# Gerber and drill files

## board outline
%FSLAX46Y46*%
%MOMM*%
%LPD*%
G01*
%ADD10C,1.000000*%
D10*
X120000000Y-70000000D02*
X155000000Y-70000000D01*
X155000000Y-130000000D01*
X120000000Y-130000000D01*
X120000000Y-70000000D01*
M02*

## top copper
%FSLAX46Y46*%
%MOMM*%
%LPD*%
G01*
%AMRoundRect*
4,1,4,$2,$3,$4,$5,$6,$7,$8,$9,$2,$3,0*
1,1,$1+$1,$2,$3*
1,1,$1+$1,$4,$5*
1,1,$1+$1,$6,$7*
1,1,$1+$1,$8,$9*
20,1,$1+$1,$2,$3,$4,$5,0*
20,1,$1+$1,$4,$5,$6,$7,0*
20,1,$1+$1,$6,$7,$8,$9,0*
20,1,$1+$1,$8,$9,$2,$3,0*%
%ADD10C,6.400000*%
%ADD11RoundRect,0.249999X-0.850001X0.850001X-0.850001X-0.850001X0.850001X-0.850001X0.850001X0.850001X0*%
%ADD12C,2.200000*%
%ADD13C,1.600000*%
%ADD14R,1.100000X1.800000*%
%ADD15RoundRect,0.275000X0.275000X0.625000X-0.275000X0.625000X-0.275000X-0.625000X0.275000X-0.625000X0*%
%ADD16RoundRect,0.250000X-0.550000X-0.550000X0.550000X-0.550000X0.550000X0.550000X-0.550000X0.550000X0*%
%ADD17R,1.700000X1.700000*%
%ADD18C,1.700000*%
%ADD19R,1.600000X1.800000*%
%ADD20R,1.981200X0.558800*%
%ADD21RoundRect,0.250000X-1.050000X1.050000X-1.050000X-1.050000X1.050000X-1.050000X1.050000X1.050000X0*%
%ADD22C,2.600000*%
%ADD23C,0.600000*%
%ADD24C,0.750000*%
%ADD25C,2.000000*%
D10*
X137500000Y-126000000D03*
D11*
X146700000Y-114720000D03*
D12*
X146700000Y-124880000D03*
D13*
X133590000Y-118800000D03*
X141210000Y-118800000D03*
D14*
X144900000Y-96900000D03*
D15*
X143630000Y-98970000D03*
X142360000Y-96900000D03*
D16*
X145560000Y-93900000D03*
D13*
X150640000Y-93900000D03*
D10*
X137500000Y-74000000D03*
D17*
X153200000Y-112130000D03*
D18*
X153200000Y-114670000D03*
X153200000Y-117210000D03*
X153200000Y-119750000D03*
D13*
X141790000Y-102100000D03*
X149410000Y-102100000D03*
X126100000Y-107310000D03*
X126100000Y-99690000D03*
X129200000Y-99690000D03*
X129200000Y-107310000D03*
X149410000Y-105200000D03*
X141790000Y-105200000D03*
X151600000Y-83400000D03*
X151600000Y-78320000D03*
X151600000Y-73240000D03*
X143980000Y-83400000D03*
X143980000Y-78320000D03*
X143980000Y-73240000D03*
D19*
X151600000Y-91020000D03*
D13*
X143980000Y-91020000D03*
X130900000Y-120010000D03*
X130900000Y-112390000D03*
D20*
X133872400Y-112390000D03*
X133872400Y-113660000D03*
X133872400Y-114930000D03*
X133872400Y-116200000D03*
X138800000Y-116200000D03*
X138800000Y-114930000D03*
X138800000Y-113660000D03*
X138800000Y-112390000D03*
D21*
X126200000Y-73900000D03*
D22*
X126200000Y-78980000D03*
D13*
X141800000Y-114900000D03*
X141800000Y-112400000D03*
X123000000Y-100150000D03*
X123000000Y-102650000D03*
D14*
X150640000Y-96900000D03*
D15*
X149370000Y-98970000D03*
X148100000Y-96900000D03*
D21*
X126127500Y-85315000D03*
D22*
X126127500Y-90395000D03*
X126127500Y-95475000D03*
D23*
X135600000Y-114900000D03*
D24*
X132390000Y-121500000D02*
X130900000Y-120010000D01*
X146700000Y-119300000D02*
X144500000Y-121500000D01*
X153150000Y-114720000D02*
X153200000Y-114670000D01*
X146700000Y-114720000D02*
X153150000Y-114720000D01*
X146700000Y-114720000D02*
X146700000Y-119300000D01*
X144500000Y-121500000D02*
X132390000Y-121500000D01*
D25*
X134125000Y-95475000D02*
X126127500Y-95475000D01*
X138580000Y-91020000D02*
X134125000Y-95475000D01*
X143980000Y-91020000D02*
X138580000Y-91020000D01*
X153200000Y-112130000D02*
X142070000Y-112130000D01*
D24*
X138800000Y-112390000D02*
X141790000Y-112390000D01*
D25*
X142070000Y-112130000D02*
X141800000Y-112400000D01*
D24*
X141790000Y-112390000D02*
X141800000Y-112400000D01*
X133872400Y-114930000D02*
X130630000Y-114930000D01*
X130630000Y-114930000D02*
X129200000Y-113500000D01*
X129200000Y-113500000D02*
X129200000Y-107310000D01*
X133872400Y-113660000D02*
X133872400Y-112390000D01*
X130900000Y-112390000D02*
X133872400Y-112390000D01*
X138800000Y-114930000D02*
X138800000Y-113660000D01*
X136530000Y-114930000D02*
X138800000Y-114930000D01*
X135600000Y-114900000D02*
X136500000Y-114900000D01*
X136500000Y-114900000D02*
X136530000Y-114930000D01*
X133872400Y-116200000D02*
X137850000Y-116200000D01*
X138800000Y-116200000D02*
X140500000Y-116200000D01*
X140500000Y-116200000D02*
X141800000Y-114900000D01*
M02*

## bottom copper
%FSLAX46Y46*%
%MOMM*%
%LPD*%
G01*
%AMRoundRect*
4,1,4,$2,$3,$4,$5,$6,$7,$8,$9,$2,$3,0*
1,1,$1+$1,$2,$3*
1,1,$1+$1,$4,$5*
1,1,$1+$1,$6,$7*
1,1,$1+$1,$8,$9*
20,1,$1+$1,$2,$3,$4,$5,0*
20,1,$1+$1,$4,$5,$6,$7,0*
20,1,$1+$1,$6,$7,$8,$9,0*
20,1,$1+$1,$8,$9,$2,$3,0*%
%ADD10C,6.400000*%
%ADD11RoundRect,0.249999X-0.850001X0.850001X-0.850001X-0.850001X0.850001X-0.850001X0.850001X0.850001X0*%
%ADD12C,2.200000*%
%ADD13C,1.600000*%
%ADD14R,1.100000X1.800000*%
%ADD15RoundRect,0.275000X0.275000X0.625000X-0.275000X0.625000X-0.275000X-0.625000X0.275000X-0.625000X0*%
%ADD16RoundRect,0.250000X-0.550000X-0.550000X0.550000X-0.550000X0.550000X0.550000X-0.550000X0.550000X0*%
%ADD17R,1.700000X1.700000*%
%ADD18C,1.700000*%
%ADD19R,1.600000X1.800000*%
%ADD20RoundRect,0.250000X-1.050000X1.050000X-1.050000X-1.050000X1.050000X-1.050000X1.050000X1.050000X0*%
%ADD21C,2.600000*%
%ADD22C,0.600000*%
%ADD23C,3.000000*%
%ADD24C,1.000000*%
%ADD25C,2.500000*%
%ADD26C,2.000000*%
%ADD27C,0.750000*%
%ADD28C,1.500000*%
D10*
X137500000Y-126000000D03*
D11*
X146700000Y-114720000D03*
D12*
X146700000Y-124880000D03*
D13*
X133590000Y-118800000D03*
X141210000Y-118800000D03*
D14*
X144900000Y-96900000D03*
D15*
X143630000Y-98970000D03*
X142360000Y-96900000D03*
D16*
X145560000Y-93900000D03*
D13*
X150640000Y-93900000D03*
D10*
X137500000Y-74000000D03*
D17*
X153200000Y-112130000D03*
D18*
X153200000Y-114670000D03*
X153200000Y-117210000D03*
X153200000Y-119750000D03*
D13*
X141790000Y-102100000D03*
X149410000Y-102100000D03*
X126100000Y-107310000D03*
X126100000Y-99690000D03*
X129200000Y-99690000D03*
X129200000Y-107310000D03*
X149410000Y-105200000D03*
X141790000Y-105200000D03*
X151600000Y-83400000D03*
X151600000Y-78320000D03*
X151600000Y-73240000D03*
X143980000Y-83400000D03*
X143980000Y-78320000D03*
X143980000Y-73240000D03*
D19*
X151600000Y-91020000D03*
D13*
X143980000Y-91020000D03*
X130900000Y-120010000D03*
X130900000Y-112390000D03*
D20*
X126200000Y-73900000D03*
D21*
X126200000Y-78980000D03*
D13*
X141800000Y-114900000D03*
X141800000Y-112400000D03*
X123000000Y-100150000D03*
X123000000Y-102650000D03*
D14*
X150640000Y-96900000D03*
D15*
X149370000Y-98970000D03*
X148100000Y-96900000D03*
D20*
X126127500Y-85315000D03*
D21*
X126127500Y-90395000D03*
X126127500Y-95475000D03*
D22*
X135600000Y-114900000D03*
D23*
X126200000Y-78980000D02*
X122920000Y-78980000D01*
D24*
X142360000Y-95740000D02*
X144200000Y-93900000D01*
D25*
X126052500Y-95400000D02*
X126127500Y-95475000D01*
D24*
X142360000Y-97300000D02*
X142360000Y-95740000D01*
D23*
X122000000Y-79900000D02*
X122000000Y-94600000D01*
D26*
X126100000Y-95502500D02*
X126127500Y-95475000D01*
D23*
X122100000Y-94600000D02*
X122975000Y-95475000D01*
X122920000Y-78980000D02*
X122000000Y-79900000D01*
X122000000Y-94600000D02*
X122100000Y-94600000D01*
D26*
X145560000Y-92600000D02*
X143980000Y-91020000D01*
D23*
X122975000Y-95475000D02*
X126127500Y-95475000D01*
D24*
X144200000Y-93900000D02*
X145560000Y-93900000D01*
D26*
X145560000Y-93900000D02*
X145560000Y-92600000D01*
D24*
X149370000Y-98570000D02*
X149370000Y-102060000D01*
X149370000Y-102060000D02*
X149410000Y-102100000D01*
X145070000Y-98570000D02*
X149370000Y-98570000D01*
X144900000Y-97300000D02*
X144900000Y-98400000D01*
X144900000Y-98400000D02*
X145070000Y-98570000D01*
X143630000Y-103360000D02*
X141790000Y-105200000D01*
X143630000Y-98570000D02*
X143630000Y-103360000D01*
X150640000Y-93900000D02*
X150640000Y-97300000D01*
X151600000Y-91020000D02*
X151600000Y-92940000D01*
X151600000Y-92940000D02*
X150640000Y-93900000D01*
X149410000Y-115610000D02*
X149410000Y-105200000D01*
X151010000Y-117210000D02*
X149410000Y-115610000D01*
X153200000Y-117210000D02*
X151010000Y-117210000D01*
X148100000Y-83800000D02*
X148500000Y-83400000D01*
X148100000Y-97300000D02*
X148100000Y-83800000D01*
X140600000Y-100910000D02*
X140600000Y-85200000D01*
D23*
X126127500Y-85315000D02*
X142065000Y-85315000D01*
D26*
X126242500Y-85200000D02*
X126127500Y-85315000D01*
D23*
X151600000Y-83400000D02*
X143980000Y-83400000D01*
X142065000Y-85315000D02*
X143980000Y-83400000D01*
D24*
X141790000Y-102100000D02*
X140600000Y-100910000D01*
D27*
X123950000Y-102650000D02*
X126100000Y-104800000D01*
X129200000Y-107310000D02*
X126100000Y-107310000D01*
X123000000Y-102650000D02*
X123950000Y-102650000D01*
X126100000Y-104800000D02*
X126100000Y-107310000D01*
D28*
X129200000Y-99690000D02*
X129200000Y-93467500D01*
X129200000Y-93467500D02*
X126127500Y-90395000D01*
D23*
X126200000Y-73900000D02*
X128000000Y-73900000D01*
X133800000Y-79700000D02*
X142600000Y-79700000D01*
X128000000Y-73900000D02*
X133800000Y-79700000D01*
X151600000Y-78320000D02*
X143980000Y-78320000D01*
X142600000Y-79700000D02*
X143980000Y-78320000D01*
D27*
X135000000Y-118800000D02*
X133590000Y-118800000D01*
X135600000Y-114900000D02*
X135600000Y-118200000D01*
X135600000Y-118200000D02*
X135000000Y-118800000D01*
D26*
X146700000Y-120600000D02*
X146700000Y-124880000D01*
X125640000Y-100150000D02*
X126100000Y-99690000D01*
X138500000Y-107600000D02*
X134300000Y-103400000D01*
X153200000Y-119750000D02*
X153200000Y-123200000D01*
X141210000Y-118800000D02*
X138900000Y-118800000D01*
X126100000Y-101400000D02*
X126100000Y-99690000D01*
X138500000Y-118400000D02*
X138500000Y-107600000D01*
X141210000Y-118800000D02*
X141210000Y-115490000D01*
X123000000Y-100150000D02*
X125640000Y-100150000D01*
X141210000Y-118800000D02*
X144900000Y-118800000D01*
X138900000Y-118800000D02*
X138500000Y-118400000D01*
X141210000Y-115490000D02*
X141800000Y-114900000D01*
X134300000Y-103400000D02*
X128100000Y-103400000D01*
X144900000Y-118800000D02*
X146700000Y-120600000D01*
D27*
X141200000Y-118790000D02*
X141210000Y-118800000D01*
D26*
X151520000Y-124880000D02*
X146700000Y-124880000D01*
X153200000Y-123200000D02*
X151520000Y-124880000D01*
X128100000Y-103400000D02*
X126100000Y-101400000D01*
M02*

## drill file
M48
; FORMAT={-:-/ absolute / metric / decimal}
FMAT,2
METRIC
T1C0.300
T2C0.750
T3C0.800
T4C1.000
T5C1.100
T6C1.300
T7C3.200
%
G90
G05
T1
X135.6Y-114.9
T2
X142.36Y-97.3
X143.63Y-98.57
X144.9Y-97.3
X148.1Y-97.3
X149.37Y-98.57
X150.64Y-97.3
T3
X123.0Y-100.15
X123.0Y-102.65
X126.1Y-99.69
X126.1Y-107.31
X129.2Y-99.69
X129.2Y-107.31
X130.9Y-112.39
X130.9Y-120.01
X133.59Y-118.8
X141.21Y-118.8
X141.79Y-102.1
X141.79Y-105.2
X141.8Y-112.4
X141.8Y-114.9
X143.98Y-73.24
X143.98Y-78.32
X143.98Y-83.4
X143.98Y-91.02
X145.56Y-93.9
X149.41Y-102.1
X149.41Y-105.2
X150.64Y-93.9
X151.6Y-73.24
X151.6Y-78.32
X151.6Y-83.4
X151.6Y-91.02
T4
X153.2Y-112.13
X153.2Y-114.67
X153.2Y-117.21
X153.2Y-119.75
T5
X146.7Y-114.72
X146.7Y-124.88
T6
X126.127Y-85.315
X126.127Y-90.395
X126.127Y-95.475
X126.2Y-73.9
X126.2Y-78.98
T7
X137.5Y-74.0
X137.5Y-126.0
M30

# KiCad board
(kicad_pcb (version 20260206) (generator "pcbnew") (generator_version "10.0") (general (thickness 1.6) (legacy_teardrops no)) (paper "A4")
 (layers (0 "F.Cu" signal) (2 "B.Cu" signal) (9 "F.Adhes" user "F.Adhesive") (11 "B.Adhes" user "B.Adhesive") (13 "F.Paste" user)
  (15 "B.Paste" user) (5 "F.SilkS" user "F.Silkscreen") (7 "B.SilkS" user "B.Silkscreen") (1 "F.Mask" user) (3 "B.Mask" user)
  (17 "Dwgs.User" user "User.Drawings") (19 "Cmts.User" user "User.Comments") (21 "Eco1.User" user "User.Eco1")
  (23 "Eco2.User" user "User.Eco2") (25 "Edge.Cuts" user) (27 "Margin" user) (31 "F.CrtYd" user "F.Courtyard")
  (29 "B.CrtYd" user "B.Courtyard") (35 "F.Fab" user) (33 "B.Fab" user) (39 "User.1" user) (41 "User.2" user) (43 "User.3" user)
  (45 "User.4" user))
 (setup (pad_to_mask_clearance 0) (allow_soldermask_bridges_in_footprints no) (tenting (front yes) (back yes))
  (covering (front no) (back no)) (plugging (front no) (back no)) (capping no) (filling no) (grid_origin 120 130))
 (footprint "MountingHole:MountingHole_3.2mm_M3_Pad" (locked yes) (layer "F.Cu") (at 137.5 126)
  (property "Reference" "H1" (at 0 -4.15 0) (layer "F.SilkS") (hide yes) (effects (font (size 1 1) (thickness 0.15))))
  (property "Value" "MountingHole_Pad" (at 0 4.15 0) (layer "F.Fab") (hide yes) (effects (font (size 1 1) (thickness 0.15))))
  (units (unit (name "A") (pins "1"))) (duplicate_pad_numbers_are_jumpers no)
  (pad "1" thru_hole circle (at 0 0) (size 6.4 6.4) (drill 3.2) (layers "*.Cu" "*.Mask") (remove_unused_layers no)
   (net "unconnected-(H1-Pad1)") (zone_connect 2)))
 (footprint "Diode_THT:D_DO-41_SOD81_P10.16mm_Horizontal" (layer "F.Cu") (at 146.7 114.72 -90)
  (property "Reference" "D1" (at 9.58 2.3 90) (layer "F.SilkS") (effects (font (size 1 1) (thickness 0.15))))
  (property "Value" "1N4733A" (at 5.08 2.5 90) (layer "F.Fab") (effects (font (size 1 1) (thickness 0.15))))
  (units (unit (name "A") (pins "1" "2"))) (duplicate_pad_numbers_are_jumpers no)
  (pad "1" thru_hole roundrect (at 0 0 270) (size 2.2 2.2) (drill 1.1) (layers "*.Cu" "*.Mask") (remove_unused_layers no)
   (roundrect_rratio 0.113636) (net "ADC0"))
  (pad "2" thru_hole circle (at 10.16 0 270) (size 2.2 2.2) (drill 1.1) (layers "*.Cu" "*.Mask") (remove_unused_layers no) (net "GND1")))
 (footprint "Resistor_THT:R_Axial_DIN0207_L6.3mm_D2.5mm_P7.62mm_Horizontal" (layer "F.Cu") (at 133.59 118.8)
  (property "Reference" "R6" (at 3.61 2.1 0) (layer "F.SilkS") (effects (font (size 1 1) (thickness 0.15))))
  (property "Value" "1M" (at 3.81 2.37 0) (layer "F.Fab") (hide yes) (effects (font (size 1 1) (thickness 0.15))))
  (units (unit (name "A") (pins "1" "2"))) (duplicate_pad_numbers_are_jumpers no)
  (pad "1" thru_hole circle (at 0 0) (size 1.6 1.6) (drill 0.8) (layers "*.Cu" "*.Mask") (remove_unused_layers no) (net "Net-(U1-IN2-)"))
  (pad "2" thru_hole circle (at 7.62 0) (size 1.6 1.6) (drill 0.8) (layers "*.Cu" "*.Mask") (remove_unused_layers no) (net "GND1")))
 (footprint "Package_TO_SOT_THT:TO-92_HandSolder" (layer "F.Cu") (at 144.9 97.3 180)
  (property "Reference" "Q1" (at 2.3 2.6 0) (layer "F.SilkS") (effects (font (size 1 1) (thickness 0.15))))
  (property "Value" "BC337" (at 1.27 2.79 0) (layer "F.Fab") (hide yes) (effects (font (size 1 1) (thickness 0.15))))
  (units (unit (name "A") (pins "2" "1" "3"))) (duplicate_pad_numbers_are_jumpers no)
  (pad "1" thru_hole rect (at 0 0 180) (size 1.1 1.8) (drill 0.75 (offset 0 0.4)) (layers "*.Cu" "*.Mask") (remove_unused_layers no)
   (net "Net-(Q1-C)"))
  (pad "2" thru_hole roundrect (at 1.27 -1.27 180) (size 1.1 1.8) (drill 0.75 (offset 0 -0.4)) (layers "*.Cu" "*.Mask")
   (remove_unused_layers no) (roundrect_rratio 0.25) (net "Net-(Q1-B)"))
  (pad "3" thru_hole roundrect (at 2.54 0 180) (size 1.1 1.8) (drill 0.75 (offset 0 0.4)) (layers "*.Cu" "*.Mask") (remove_unused_layers no)
   (roundrect_rratio 0.25) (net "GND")))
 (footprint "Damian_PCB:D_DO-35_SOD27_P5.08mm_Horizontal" (layer "F.Cu") (at 148.1 93.9)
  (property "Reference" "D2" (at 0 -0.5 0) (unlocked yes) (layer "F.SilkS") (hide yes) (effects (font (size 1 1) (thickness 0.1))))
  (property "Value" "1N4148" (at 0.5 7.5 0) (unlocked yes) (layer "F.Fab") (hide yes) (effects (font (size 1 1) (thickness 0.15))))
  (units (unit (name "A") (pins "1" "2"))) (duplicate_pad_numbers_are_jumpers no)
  (pad "1" thru_hole roundrect (at -2.54 0) (size 1.6 1.6) (drill 0.8) (layers "*.Cu" "*.Mask") (remove_unused_layers no)
   (roundrect_rratio 0.15625) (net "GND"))
  (pad "2" thru_hole circle (at 2.54 0) (size 1.6 1.6) (drill 0.8) (layers "*.Cu" "*.Mask") (remove_unused_layers no) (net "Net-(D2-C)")))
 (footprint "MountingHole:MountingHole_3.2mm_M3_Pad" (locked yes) (layer "F.Cu") (at 137.5 74)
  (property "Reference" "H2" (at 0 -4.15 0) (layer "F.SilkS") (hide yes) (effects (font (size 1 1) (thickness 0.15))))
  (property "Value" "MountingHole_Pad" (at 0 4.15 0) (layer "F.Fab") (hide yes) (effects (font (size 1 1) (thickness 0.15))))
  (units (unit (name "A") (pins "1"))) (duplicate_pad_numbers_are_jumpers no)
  (pad "1" thru_hole circle (at 0 0) (size 6.4 6.4) (drill 3.2) (layers "*.Cu" "*.Mask") (remove_unused_layers no)
   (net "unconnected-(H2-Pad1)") (zone_connect 2)))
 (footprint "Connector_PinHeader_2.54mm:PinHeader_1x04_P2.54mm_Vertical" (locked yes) (layer "F.Cu") (at 153.2 112.13)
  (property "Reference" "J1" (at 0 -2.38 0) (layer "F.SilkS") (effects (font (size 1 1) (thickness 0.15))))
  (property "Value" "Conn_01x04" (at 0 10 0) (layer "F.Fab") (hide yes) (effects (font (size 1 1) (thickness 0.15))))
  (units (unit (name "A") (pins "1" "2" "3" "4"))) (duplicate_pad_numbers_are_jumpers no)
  (pad "1" thru_hole rect (at 0 0) (size 1.7 1.7) (drill 1) (layers "*.Cu" "*.Mask") (remove_unused_layers no) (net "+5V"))
  (pad "2" thru_hole circle (at 0 2.54) (size 1.7 1.7) (drill 1) (layers "*.Cu" "*.Mask") (remove_unused_layers no) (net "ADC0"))
  (pad "3" thru_hole circle (at 0 5.08) (size 1.7 1.7) (drill 1) (layers "*.Cu" "*.Mask") (remove_unused_layers no) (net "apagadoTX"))
  (pad "4" thru_hole circle (at 0 7.62) (size 1.7 1.7) (drill 1) (layers "*.Cu" "*.Mask") (remove_unused_layers no) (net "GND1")))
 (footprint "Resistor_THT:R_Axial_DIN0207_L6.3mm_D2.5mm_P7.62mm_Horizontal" (layer "F.Cu") (at 141.79 102.1)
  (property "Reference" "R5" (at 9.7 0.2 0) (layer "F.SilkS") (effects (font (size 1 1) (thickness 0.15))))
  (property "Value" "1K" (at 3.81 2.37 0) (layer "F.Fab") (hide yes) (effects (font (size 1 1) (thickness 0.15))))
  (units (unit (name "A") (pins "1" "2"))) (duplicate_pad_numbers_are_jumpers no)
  (pad "1" thru_hole circle (at 0 0) (size 1.6 1.6) (drill 0.8) (layers "*.Cu" "*.Mask") (remove_unused_layers no) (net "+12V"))
  (pad "2" thru_hole circle (at 7.62 0) (size 1.6 1.6) (drill 0.8) (layers "*.Cu" "*.Mask") (remove_unused_layers no) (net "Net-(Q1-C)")))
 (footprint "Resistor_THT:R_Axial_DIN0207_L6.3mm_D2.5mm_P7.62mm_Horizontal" (layer "F.Cu") (at 126.1 107.31 90)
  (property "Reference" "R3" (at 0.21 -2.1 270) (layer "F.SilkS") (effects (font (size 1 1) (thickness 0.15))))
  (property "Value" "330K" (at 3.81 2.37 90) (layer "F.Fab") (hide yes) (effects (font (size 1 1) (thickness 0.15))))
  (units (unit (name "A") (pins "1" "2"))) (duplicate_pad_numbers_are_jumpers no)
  (pad "1" thru_hole circle (at 0 0 90) (size 1.6 1.6) (drill 0.8) (layers "*.Cu" "*.Mask") (remove_unused_layers no) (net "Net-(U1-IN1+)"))
  (pad "2" thru_hole circle (at 7.62 0 90) (size 1.6 1.6) (drill 0.8) (layers "*.Cu" "*.Mask") (remove_unused_layers no) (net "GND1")))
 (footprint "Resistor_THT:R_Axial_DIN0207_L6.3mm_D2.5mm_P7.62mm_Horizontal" (layer "F.Cu") (at 129.2 99.69 -90)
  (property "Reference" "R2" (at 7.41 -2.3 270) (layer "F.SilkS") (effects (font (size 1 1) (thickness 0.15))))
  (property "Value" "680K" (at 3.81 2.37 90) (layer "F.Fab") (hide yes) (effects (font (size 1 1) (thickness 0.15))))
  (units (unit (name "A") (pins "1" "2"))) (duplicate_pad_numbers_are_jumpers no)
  (pad "1" thru_hole circle (at 0 0 270) (size 1.6 1.6) (drill 0.8) (layers "*.Cu" "*.Mask") (remove_unused_layers no) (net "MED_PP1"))
  (pad "2" thru_hole circle (at 7.62 0 270) (size 1.6 1.6) (drill 0.8) (layers "*.Cu" "*.Mask") (remove_unused_layers no)
   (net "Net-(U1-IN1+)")))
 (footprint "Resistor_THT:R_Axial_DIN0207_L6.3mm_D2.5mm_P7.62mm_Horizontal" (layer "F.Cu") (at 149.41 105.2 180)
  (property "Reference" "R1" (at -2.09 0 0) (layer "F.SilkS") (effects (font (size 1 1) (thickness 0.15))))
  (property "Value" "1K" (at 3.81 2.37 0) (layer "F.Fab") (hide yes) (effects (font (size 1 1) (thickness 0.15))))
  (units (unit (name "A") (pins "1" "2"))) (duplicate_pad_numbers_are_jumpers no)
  (pad "1" thru_hole circle (at 0 0 180) (size 1.6 1.6) (drill 0.8) (layers "*.Cu" "*.Mask") (remove_unused_layers no) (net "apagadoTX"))
  (pad "2" thru_hole circle (at 7.62 0 180) (size 1.6 1.6) (drill 0.8) (layers "*.Cu" "*.Mask") (remove_unused_layers no) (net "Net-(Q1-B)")))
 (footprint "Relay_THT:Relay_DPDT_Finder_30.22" (layer "F.Cu") (at 151.6 91.02 90)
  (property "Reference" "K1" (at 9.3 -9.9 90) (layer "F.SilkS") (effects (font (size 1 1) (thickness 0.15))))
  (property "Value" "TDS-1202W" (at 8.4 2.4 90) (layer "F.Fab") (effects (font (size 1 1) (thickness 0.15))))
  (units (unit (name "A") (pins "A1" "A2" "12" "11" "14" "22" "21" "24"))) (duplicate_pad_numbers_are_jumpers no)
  (pad "11" thru_hole circle (at 7.62 0 180) (size 1.6 1.6) (drill 0.8) (layers "*.Cu" "*.Mask") (remove_unused_layers no) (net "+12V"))
  (pad "12" thru_hole circle (at 12.7 0 180) (size 1.6 1.6) (drill 0.8) (layers "*.Cu" "*.Mask") (remove_unused_layers no) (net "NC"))
  (pad "14" thru_hole circle (at 17.78 0 180) (size 1.6 1.6) (drill 0.8) (layers "*.Cu" "*.Mask") (remove_unused_layers no)
   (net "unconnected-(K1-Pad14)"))
  (pad "21" thru_hole circle (at 7.62 -7.62 180) (size 1.6 1.6) (drill 0.8) (layers "*.Cu" "*.Mask") (remove_unused_layers no) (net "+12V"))
  (pad "22" thru_hole circle (at 12.7 -7.62 180) (size 1.6 1.6) (drill 0.8) (layers "*.Cu" "*.Mask") (remove_unused_layers no) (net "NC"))
  (pad "24" thru_hole circle (at 17.78 -7.62 270) (size 1.6 1.6) (drill 0.8) (layers "*.Cu" "*.Mask") (remove_unused_layers no)
   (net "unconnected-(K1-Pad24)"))
  (pad "A1" thru_hole rect (at 0 0 180) (size 1.6 1.8) (drill 0.8) (layers "*.Cu" "*.Mask") (remove_unused_layers no) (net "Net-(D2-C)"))
  (pad "A2" thru_hole circle (at 0 -7.62 180) (size 1.6 1.6) (drill 0.8) (layers "*.Cu" "*.Mask") (remove_unused_layers no) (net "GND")))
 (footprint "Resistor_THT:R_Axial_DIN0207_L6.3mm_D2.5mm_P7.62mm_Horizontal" (layer "F.Cu") (at 130.9 120.01 90)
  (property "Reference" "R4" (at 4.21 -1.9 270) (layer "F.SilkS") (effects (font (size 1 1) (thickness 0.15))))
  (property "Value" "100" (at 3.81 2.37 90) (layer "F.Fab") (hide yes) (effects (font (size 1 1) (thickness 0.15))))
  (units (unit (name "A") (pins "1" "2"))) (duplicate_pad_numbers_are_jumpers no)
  (pad "1" thru_hole circle (at 0 0 90) (size 1.6 1.6) (drill 0.8) (layers "*.Cu" "*.Mask") (remove_unused_layers no) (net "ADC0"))
  (pad "2" thru_hole circle (at 7.62 0 90) (size 1.6 1.6) (drill 0.8) (layers "*.Cu" "*.Mask") (remove_unused_layers no)
   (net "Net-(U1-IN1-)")))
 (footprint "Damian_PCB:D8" (layer "F.Cu") (at 136.3362 114.295)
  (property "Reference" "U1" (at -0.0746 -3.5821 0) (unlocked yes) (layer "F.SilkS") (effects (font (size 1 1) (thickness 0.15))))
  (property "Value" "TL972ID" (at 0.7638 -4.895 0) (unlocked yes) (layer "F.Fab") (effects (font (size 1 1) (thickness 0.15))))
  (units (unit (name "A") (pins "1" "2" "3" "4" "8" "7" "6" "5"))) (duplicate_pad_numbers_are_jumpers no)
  (pad "1" smd rect (at -2.4638 -1.905) (size 1.9812 0.5588) (layers "F.Cu" "F.Mask" "F.Paste") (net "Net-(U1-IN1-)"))
  (pad "2" smd rect (at -2.4638 -0.635) (size 1.9812 0.5588) (layers "F.Cu" "F.Mask" "F.Paste") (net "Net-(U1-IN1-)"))
  (pad "3" smd rect (at -2.4638 0.635) (size 1.9812 0.5588) (layers "F.Cu" "F.Mask" "F.Paste") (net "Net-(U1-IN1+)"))
  (pad "4" smd rect (at -2.4638 1.905) (size 1.9812 0.5588) (layers "F.Cu" "F.Mask" "F.Paste") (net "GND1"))
  (pad "5" smd rect (at 2.4638 1.905) (size 1.9812 0.5588) (layers "F.Cu" "F.Mask" "F.Paste") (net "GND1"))
  (pad "6" smd rect (at 2.4638 0.635) (size 1.9812 0.5588) (layers "F.Cu" "F.Mask" "F.Paste") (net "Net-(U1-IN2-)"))
  (pad "7" smd rect (at 2.4638 -0.635) (size 1.9812 0.5588) (layers "F.Cu" "F.Mask" "F.Paste") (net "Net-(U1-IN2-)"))
  (pad "8" smd rect (at 2.4638 -1.905) (size 1.9812 0.5588) (layers "F.Cu" "F.Mask" "F.Paste") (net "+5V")))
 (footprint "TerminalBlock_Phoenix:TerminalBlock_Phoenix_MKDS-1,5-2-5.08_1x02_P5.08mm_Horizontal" (layer "F.Cu") (at 126.2 73.9 -90)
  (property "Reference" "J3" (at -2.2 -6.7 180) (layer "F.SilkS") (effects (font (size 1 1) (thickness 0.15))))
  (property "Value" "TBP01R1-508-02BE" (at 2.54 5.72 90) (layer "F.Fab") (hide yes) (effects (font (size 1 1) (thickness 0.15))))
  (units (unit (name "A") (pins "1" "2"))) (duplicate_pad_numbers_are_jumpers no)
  (pad "1" thru_hole roundrect (at 0 0 270) (size 2.6 2.6) (drill 1.3) (layers "*.Cu" "*.Mask") (remove_unused_layers no)
   (roundrect_rratio 0.096154) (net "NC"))
  (pad "2" thru_hole circle (at 5.08 0 270) (size 2.6 2.6) (drill 1.3) (layers "*.Cu" "*.Mask") (remove_unused_layers no) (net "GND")))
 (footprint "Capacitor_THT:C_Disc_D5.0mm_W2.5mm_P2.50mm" (layer "F.Cu") (at 141.8 114.9 90)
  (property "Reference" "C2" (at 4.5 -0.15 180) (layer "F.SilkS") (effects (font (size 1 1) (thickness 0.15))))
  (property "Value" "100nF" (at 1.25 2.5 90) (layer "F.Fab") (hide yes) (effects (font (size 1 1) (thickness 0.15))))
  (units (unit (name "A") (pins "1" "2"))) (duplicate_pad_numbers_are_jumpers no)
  (pad "1" thru_hole circle (at 0 0 90) (size 1.6 1.6) (drill 0.8) (layers "*.Cu" "*.Mask") (remove_unused_layers no) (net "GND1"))
  (pad "2" thru_hole circle (at 2.5 0 90) (size 1.6 1.6) (drill 0.8) (layers "*.Cu" "*.Mask") (remove_unused_layers no) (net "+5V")))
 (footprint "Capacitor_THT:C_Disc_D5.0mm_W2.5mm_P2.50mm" (layer "F.Cu") (at 123 100.15 -90)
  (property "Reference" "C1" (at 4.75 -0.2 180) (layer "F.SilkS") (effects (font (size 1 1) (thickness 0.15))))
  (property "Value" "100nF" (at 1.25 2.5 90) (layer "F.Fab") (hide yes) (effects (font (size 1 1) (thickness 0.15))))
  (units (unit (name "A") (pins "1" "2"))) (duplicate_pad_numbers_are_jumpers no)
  (pad "1" thru_hole circle (at 0 0 270) (size 1.6 1.6) (drill 0.8) (layers "*.Cu" "*.Mask") (remove_unused_layers no) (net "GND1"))
  (pad "2" thru_hole circle (at 2.5 0 270) (size 1.6 1.6) (drill 0.8) (layers "*.Cu" "*.Mask") (remove_unused_layers no)
   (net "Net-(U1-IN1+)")))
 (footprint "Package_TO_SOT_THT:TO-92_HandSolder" (layer "F.Cu") (at 150.64 97.3 180)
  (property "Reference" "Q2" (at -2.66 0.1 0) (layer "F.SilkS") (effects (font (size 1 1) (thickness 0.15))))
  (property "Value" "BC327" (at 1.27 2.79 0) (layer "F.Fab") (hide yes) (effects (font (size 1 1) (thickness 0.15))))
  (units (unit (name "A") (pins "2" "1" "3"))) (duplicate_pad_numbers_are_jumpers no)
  (pad "1" thru_hole rect (at 0 0 180) (size 1.1 1.8) (drill 0.75 (offset 0 0.4)) (layers "*.Cu" "*.Mask") (remove_unused_layers no)
   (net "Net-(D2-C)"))
  (pad "2" thru_hole roundrect (at 1.27 -1.27 180) (size 1.1 1.8) (drill 0.75 (offset 0 -0.4)) (layers "*.Cu" "*.Mask")
   (remove_unused_layers no) (roundrect_rratio 0.25) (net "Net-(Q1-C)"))
  (pad "3" thru_hole roundrect (at 2.54 0 180) (size 1.1 1.8) (drill 0.75 (offset 0 0.4)) (layers "*.Cu" "*.Mask") (remove_unused_layers no)
   (roundrect_rratio 0.25) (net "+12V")))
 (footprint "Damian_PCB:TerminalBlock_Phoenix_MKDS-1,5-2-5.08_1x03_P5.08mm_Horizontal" (layer "F.Cu") (at 126.1275 85.315 -90)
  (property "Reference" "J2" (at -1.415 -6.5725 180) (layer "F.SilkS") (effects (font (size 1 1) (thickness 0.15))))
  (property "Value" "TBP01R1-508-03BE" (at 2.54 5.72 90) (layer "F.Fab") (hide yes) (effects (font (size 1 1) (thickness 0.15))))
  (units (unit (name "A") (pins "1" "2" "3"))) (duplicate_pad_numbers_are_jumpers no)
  (pad "1" thru_hole roundrect (at 0 0 270) (size 2.6 2.6) (drill 1.3) (layers "*.Cu" "*.Mask") (remove_unused_layers no)
   (roundrect_rratio 0.096154) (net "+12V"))
  (pad "2" thru_hole circle (at 5.08 0 270) (size 2.6 2.6) (drill 1.3) (layers "*.Cu" "*.Mask") (remove_unused_layers no) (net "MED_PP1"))
  (pad "3" thru_hole circle (at 10.16 0 270) (size 2.6 2.6) (drill 1.3) (layers "*.Cu" "*.Mask") (remove_unused_layers no) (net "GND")))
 (gr_rect (start 120 70) (end 155 130) (stroke (width 1) (type solid)) (fill no) (locked yes) (layer "Edge.Cuts"))
 (segment (start 132.39 121.5) (end 130.9 120.01) (width 0.75) (layer "F.Cu") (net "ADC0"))
 (segment (start 146.7 119.3) (end 144.5 121.5) (width 0.75) (layer "F.Cu") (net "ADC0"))
 (segment (start 153.15 114.72) (end 153.2 114.67) (width 0.75) (layer "F.Cu") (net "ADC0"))
 (segment (start 146.7 114.72) (end 153.15 114.72) (width 0.75) (layer "F.Cu") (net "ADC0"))
 (segment (start 146.7 114.72) (end 146.7 119.3) (width 0.75) (layer "F.Cu") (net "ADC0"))
 (segment (start 144.5 121.5) (end 132.39 121.5) (width 0.75) (layer "F.Cu") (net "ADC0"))
 (segment (start 134.125 95.475) (end 126.1275 95.475) (width 2) (layer "F.Cu") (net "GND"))
 (segment (start 138.58 91.02) (end 134.125 95.475) (width 2) (layer "F.Cu") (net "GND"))
 (segment (start 143.98 91.02) (end 138.58 91.02) (width 2) (layer "F.Cu") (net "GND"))
 (segment (start 126.2 78.98) (end 122.92 78.98) (width 3) (layer "B.Cu") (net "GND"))
 (segment (start 142.36 95.74) (end 144.2 93.9) (width 1) (layer "B.Cu") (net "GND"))
 (segment (start 126.0525 95.4) (end 126.1275 95.475) (width 2.5) (layer "B.Cu") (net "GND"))
 (segment (start 142.36 97.3) (end 142.36 95.74) (width 1) (layer "B.Cu") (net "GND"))
 (segment (start 122 79.9) (end 122 94.6) (width 3) (layer "B.Cu") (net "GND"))
 (segment (start 126.1 95.5025) (end 126.1275 95.475) (width 2) (layer "B.Cu") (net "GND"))
 (segment (start 122.1 94.6) (end 122.975 95.475) (width 3) (layer "B.Cu") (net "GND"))
 (segment (start 122.92 78.98) (end 122 79.9) (width 3) (layer "B.Cu") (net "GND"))
 (segment (start 122 94.6) (end 122.1 94.6) (width 3) (layer "B.Cu") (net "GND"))
 (segment (start 145.56 92.6) (end 143.98 91.02) (width 2) (layer "B.Cu") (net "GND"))
 (segment (start 122.975 95.475) (end 126.1275 95.475) (width 3) (layer "B.Cu") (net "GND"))
 (segment (start 144.2 93.9) (end 145.56 93.9) (width 1) (layer "B.Cu") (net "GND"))
 (segment (start 145.56 93.9) (end 145.56 92.6) (width 2) (layer "B.Cu") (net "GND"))
 (segment (start 149.37 98.57) (end 149.37 102.06) (width 1) (layer "B.Cu") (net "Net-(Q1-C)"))
 (segment (start 149.37 102.06) (end 149.41 102.1) (width 1) (layer "B.Cu") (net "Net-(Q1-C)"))
 (segment (start 145.07 98.57) (end 149.37 98.57) (width 1) (layer "B.Cu") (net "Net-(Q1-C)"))
 (segment (start 144.9 97.3) (end 144.9 98.4) (width 1) (layer "B.Cu") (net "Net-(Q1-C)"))
 (segment (start 144.9 98.4) (end 145.07 98.57) (width 1) (layer "B.Cu") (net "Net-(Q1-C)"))
 (segment (start 143.63 103.36) (end 141.79 105.2) (width 1) (layer "B.Cu") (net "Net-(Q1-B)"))
 (segment (start 143.63 98.57) (end 143.63 103.36) (width 1) (layer "B.Cu") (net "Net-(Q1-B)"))
 (segment (start 150.64 93.9) (end 150.64 97.3) (width 1) (layer "B.Cu") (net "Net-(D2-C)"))
 (segment (start 151.6 91.02) (end 151.6 92.94) (width 1) (layer "B.Cu") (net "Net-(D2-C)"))
 (segment (start 151.6 92.94) (end 150.64 93.9) (width 1) (layer "B.Cu") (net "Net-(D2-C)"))
 (segment (start 153.2 112.13) (end 142.07 112.13) (width 2) (layer "F.Cu") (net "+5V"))
 (segment (start 138.8 112.39) (end 141.79 112.39) (width 0.75) (layer "F.Cu") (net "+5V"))
 (segment (start 142.07 112.13) (end 141.8 112.4) (width 2) (layer "F.Cu") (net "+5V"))
 (segment (start 141.79 112.39) (end 141.8 112.4) (width 0.75) (layer "F.Cu") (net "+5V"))
 (segment (start 149.41 115.61) (end 149.41 105.2) (width 1) (layer "B.Cu") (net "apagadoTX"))
 (segment (start 151.01 117.21) (end 149.41 115.61) (width 1) (layer "B.Cu") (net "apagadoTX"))
 (segment (start 153.2 117.21) (end 151.01 117.21) (width 1) (layer "B.Cu") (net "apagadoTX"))
 (segment (start 148.1 83.8) (end 148.5 83.4) (width 1) (layer "B.Cu") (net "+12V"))
 (segment (start 148.1 97.3) (end 148.1 83.8) (width 1) (layer "B.Cu") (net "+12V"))
 (segment (start 140.6 100.91) (end 140.6 85.2) (width 1) (layer "B.Cu") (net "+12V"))
 (segment (start 126.1275 85.315) (end 142.065 85.315) (width 3) (layer "B.Cu") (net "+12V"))
 (segment (start 126.2425 85.2) (end 126.1275 85.315) (width 2) (layer "B.Cu") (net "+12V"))
 (segment (start 151.6 83.4) (end 143.98 83.4) (width 3) (layer "B.Cu") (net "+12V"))
 (segment (start 142.065 85.315) (end 143.98 83.4) (width 3) (layer "B.Cu") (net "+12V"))
 (segment (start 141.79 102.1) (end 140.6 100.91) (width 1) (layer "B.Cu") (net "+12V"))
 (segment (start 133.8724 114.93) (end 130.63 114.93) (width 0.75) (layer "F.Cu") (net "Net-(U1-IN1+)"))
 (segment (start 130.63 114.93) (end 129.2 113.5) (width 0.75) (layer "F.Cu") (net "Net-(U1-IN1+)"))
 (segment (start 129.2 113.5) (end 129.2 107.31) (width 0.75) (layer "F.Cu") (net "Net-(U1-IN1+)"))
 (segment (start 123.95 102.65) (end 126.1 104.8) (width 0.75) (layer "B.Cu") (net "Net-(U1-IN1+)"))
 (segment (start 129.2 107.31) (end 126.1 107.31) (width 0.75) (layer "B.Cu") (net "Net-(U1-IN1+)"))
 (segment (start 123 102.65) (end 123.95 102.65) (width 0.75) (layer "B.Cu") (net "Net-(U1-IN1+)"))
 (segment (start 126.1 104.8) (end 126.1 107.31) (width 0.75) (layer "B.Cu") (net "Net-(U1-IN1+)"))
 (segment (start 129.2 99.69) (end 129.2 93.4675) (width 1.5) (layer "B.Cu") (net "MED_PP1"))
 (segment (start 129.2 93.4675) (end 126.1275 90.395) (width 1.5) (layer "B.Cu") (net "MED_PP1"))
 (segment (start 126.2 73.9) (end 128 73.9) (width 3) (layer "B.Cu") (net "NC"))
 (segment (start 133.8 79.7) (end 142.6 79.7) (width 3) (layer "B.Cu") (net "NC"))
 (segment (start 128 73.9) (end 133.8 79.7) (width 3) (layer "B.Cu") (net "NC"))
 (segment (start 151.6 78.32) (end 143.98 78.32) (width 3) (layer "B.Cu") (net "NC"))
 (segment (start 142.6 79.7) (end 143.98 78.32) (width 3) (layer "B.Cu") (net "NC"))
 (segment (start 133.8724 113.66) (end 133.8724 112.39) (width 0.75) (layer "F.Cu") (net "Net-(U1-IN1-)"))
 (segment (start 130.9 112.39) (end 133.8724 112.39) (width 0.75) (layer "F.Cu") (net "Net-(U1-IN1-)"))
 (segment (start 138.8 114.93) (end 138.8 113.66) (width 0.75) (layer "F.Cu") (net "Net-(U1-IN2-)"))
 (segment (start 136.53 114.93) (end 138.8 114.93) (width 0.75) (layer "F.Cu") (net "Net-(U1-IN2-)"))
 (segment (start 135.6 114.9) (end 136.5 114.9) (width 0.75) (layer "F.Cu") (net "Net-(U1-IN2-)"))
 (segment (start 136.5 114.9) (end 136.53 114.93) (width 0.75) (layer "F.Cu") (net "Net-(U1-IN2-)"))
 (via (at 135.6 114.9) (size 0.6) (drill 0.3) (layers "F.Cu" "B.Cu") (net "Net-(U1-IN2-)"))
 (segment (start 135 118.8) (end 133.59 118.8) (width 0.75) (layer "B.Cu") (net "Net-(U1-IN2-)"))
 (segment (start 135.6 114.9) (end 135.6 118.2) (width 0.75) (layer "B.Cu") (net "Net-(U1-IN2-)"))
 (segment (start 135.6 118.2) (end 135 118.8) (width 0.75) (layer "B.Cu") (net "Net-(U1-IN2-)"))
 (segment (start 133.8724 116.2) (end 137.85 116.2) (width 0.75) (layer "F.Cu") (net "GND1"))
 (segment (start 138.8 116.2) (end 140.5 116.2) (width 0.75) (layer "F.Cu") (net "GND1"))
 (segment (start 140.5 116.2) (end 141.8 114.9) (width 0.75) (layer "F.Cu") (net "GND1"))
 (segment (start 146.7 120.6) (end 146.7 124.88) (width 2) (layer "B.Cu") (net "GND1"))
 (segment (start 125.64 100.15) (end 126.1 99.69) (width 2) (layer "B.Cu") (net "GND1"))
 (segment (start 138.5 107.6) (end 134.3 103.4) (width 2) (layer "B.Cu") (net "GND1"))
 (segment (start 153.2 119.75) (end 153.2 123.2) (width 2) (layer "B.Cu") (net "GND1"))
 (segment (start 141.21 118.8) (end 138.9 118.8) (width 2) (layer "B.Cu") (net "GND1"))
 (segment (start 126.1 101.4) (end 126.1 99.69) (width 2) (layer "B.Cu") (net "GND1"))
 (segment (start 138.5 118.4) (end 138.5 107.6) (width 2) (layer "B.Cu") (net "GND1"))
 (segment (start 141.21 118.8) (end 141.21 115.49) (width 2) (layer "B.Cu") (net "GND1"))
 (segment (start 123 100.15) (end 125.64 100.15) (width 2) (layer "B.Cu") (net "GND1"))
 (segment (start 141.21 118.8) (end 144.9 118.8) (width 2) (layer "B.Cu") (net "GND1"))
 (segment (start 138.9 118.8) (end 138.5 118.4) (width 2) (layer "B.Cu") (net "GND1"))
 (segment (start 141.21 115.49) (end 141.8 114.9) (width 2) (layer "B.Cu") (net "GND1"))
 (segment (start 134.3 103.4) (end 128.1 103.4) (width 2) (layer "B.Cu") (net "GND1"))
 (segment (start 144.9 118.8) (end 146.7 120.6) (width 2) (layer "B.Cu") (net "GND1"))
 (segment (start 141.2 118.79) (end 141.21 118.8) (width 0.75) (layer "B.Cu") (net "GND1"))
 (segment (start 151.52 124.88) (end 146.7 124.88) (width 2) (layer "B.Cu") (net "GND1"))
 (segment (start 153.2 123.2) (end 151.52 124.88) (width 2) (layer "B.Cu") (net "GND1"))
 (segment (start 128.1 103.4) (end 126.1 101.4) (width 2) (layer "B.Cu") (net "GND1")))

